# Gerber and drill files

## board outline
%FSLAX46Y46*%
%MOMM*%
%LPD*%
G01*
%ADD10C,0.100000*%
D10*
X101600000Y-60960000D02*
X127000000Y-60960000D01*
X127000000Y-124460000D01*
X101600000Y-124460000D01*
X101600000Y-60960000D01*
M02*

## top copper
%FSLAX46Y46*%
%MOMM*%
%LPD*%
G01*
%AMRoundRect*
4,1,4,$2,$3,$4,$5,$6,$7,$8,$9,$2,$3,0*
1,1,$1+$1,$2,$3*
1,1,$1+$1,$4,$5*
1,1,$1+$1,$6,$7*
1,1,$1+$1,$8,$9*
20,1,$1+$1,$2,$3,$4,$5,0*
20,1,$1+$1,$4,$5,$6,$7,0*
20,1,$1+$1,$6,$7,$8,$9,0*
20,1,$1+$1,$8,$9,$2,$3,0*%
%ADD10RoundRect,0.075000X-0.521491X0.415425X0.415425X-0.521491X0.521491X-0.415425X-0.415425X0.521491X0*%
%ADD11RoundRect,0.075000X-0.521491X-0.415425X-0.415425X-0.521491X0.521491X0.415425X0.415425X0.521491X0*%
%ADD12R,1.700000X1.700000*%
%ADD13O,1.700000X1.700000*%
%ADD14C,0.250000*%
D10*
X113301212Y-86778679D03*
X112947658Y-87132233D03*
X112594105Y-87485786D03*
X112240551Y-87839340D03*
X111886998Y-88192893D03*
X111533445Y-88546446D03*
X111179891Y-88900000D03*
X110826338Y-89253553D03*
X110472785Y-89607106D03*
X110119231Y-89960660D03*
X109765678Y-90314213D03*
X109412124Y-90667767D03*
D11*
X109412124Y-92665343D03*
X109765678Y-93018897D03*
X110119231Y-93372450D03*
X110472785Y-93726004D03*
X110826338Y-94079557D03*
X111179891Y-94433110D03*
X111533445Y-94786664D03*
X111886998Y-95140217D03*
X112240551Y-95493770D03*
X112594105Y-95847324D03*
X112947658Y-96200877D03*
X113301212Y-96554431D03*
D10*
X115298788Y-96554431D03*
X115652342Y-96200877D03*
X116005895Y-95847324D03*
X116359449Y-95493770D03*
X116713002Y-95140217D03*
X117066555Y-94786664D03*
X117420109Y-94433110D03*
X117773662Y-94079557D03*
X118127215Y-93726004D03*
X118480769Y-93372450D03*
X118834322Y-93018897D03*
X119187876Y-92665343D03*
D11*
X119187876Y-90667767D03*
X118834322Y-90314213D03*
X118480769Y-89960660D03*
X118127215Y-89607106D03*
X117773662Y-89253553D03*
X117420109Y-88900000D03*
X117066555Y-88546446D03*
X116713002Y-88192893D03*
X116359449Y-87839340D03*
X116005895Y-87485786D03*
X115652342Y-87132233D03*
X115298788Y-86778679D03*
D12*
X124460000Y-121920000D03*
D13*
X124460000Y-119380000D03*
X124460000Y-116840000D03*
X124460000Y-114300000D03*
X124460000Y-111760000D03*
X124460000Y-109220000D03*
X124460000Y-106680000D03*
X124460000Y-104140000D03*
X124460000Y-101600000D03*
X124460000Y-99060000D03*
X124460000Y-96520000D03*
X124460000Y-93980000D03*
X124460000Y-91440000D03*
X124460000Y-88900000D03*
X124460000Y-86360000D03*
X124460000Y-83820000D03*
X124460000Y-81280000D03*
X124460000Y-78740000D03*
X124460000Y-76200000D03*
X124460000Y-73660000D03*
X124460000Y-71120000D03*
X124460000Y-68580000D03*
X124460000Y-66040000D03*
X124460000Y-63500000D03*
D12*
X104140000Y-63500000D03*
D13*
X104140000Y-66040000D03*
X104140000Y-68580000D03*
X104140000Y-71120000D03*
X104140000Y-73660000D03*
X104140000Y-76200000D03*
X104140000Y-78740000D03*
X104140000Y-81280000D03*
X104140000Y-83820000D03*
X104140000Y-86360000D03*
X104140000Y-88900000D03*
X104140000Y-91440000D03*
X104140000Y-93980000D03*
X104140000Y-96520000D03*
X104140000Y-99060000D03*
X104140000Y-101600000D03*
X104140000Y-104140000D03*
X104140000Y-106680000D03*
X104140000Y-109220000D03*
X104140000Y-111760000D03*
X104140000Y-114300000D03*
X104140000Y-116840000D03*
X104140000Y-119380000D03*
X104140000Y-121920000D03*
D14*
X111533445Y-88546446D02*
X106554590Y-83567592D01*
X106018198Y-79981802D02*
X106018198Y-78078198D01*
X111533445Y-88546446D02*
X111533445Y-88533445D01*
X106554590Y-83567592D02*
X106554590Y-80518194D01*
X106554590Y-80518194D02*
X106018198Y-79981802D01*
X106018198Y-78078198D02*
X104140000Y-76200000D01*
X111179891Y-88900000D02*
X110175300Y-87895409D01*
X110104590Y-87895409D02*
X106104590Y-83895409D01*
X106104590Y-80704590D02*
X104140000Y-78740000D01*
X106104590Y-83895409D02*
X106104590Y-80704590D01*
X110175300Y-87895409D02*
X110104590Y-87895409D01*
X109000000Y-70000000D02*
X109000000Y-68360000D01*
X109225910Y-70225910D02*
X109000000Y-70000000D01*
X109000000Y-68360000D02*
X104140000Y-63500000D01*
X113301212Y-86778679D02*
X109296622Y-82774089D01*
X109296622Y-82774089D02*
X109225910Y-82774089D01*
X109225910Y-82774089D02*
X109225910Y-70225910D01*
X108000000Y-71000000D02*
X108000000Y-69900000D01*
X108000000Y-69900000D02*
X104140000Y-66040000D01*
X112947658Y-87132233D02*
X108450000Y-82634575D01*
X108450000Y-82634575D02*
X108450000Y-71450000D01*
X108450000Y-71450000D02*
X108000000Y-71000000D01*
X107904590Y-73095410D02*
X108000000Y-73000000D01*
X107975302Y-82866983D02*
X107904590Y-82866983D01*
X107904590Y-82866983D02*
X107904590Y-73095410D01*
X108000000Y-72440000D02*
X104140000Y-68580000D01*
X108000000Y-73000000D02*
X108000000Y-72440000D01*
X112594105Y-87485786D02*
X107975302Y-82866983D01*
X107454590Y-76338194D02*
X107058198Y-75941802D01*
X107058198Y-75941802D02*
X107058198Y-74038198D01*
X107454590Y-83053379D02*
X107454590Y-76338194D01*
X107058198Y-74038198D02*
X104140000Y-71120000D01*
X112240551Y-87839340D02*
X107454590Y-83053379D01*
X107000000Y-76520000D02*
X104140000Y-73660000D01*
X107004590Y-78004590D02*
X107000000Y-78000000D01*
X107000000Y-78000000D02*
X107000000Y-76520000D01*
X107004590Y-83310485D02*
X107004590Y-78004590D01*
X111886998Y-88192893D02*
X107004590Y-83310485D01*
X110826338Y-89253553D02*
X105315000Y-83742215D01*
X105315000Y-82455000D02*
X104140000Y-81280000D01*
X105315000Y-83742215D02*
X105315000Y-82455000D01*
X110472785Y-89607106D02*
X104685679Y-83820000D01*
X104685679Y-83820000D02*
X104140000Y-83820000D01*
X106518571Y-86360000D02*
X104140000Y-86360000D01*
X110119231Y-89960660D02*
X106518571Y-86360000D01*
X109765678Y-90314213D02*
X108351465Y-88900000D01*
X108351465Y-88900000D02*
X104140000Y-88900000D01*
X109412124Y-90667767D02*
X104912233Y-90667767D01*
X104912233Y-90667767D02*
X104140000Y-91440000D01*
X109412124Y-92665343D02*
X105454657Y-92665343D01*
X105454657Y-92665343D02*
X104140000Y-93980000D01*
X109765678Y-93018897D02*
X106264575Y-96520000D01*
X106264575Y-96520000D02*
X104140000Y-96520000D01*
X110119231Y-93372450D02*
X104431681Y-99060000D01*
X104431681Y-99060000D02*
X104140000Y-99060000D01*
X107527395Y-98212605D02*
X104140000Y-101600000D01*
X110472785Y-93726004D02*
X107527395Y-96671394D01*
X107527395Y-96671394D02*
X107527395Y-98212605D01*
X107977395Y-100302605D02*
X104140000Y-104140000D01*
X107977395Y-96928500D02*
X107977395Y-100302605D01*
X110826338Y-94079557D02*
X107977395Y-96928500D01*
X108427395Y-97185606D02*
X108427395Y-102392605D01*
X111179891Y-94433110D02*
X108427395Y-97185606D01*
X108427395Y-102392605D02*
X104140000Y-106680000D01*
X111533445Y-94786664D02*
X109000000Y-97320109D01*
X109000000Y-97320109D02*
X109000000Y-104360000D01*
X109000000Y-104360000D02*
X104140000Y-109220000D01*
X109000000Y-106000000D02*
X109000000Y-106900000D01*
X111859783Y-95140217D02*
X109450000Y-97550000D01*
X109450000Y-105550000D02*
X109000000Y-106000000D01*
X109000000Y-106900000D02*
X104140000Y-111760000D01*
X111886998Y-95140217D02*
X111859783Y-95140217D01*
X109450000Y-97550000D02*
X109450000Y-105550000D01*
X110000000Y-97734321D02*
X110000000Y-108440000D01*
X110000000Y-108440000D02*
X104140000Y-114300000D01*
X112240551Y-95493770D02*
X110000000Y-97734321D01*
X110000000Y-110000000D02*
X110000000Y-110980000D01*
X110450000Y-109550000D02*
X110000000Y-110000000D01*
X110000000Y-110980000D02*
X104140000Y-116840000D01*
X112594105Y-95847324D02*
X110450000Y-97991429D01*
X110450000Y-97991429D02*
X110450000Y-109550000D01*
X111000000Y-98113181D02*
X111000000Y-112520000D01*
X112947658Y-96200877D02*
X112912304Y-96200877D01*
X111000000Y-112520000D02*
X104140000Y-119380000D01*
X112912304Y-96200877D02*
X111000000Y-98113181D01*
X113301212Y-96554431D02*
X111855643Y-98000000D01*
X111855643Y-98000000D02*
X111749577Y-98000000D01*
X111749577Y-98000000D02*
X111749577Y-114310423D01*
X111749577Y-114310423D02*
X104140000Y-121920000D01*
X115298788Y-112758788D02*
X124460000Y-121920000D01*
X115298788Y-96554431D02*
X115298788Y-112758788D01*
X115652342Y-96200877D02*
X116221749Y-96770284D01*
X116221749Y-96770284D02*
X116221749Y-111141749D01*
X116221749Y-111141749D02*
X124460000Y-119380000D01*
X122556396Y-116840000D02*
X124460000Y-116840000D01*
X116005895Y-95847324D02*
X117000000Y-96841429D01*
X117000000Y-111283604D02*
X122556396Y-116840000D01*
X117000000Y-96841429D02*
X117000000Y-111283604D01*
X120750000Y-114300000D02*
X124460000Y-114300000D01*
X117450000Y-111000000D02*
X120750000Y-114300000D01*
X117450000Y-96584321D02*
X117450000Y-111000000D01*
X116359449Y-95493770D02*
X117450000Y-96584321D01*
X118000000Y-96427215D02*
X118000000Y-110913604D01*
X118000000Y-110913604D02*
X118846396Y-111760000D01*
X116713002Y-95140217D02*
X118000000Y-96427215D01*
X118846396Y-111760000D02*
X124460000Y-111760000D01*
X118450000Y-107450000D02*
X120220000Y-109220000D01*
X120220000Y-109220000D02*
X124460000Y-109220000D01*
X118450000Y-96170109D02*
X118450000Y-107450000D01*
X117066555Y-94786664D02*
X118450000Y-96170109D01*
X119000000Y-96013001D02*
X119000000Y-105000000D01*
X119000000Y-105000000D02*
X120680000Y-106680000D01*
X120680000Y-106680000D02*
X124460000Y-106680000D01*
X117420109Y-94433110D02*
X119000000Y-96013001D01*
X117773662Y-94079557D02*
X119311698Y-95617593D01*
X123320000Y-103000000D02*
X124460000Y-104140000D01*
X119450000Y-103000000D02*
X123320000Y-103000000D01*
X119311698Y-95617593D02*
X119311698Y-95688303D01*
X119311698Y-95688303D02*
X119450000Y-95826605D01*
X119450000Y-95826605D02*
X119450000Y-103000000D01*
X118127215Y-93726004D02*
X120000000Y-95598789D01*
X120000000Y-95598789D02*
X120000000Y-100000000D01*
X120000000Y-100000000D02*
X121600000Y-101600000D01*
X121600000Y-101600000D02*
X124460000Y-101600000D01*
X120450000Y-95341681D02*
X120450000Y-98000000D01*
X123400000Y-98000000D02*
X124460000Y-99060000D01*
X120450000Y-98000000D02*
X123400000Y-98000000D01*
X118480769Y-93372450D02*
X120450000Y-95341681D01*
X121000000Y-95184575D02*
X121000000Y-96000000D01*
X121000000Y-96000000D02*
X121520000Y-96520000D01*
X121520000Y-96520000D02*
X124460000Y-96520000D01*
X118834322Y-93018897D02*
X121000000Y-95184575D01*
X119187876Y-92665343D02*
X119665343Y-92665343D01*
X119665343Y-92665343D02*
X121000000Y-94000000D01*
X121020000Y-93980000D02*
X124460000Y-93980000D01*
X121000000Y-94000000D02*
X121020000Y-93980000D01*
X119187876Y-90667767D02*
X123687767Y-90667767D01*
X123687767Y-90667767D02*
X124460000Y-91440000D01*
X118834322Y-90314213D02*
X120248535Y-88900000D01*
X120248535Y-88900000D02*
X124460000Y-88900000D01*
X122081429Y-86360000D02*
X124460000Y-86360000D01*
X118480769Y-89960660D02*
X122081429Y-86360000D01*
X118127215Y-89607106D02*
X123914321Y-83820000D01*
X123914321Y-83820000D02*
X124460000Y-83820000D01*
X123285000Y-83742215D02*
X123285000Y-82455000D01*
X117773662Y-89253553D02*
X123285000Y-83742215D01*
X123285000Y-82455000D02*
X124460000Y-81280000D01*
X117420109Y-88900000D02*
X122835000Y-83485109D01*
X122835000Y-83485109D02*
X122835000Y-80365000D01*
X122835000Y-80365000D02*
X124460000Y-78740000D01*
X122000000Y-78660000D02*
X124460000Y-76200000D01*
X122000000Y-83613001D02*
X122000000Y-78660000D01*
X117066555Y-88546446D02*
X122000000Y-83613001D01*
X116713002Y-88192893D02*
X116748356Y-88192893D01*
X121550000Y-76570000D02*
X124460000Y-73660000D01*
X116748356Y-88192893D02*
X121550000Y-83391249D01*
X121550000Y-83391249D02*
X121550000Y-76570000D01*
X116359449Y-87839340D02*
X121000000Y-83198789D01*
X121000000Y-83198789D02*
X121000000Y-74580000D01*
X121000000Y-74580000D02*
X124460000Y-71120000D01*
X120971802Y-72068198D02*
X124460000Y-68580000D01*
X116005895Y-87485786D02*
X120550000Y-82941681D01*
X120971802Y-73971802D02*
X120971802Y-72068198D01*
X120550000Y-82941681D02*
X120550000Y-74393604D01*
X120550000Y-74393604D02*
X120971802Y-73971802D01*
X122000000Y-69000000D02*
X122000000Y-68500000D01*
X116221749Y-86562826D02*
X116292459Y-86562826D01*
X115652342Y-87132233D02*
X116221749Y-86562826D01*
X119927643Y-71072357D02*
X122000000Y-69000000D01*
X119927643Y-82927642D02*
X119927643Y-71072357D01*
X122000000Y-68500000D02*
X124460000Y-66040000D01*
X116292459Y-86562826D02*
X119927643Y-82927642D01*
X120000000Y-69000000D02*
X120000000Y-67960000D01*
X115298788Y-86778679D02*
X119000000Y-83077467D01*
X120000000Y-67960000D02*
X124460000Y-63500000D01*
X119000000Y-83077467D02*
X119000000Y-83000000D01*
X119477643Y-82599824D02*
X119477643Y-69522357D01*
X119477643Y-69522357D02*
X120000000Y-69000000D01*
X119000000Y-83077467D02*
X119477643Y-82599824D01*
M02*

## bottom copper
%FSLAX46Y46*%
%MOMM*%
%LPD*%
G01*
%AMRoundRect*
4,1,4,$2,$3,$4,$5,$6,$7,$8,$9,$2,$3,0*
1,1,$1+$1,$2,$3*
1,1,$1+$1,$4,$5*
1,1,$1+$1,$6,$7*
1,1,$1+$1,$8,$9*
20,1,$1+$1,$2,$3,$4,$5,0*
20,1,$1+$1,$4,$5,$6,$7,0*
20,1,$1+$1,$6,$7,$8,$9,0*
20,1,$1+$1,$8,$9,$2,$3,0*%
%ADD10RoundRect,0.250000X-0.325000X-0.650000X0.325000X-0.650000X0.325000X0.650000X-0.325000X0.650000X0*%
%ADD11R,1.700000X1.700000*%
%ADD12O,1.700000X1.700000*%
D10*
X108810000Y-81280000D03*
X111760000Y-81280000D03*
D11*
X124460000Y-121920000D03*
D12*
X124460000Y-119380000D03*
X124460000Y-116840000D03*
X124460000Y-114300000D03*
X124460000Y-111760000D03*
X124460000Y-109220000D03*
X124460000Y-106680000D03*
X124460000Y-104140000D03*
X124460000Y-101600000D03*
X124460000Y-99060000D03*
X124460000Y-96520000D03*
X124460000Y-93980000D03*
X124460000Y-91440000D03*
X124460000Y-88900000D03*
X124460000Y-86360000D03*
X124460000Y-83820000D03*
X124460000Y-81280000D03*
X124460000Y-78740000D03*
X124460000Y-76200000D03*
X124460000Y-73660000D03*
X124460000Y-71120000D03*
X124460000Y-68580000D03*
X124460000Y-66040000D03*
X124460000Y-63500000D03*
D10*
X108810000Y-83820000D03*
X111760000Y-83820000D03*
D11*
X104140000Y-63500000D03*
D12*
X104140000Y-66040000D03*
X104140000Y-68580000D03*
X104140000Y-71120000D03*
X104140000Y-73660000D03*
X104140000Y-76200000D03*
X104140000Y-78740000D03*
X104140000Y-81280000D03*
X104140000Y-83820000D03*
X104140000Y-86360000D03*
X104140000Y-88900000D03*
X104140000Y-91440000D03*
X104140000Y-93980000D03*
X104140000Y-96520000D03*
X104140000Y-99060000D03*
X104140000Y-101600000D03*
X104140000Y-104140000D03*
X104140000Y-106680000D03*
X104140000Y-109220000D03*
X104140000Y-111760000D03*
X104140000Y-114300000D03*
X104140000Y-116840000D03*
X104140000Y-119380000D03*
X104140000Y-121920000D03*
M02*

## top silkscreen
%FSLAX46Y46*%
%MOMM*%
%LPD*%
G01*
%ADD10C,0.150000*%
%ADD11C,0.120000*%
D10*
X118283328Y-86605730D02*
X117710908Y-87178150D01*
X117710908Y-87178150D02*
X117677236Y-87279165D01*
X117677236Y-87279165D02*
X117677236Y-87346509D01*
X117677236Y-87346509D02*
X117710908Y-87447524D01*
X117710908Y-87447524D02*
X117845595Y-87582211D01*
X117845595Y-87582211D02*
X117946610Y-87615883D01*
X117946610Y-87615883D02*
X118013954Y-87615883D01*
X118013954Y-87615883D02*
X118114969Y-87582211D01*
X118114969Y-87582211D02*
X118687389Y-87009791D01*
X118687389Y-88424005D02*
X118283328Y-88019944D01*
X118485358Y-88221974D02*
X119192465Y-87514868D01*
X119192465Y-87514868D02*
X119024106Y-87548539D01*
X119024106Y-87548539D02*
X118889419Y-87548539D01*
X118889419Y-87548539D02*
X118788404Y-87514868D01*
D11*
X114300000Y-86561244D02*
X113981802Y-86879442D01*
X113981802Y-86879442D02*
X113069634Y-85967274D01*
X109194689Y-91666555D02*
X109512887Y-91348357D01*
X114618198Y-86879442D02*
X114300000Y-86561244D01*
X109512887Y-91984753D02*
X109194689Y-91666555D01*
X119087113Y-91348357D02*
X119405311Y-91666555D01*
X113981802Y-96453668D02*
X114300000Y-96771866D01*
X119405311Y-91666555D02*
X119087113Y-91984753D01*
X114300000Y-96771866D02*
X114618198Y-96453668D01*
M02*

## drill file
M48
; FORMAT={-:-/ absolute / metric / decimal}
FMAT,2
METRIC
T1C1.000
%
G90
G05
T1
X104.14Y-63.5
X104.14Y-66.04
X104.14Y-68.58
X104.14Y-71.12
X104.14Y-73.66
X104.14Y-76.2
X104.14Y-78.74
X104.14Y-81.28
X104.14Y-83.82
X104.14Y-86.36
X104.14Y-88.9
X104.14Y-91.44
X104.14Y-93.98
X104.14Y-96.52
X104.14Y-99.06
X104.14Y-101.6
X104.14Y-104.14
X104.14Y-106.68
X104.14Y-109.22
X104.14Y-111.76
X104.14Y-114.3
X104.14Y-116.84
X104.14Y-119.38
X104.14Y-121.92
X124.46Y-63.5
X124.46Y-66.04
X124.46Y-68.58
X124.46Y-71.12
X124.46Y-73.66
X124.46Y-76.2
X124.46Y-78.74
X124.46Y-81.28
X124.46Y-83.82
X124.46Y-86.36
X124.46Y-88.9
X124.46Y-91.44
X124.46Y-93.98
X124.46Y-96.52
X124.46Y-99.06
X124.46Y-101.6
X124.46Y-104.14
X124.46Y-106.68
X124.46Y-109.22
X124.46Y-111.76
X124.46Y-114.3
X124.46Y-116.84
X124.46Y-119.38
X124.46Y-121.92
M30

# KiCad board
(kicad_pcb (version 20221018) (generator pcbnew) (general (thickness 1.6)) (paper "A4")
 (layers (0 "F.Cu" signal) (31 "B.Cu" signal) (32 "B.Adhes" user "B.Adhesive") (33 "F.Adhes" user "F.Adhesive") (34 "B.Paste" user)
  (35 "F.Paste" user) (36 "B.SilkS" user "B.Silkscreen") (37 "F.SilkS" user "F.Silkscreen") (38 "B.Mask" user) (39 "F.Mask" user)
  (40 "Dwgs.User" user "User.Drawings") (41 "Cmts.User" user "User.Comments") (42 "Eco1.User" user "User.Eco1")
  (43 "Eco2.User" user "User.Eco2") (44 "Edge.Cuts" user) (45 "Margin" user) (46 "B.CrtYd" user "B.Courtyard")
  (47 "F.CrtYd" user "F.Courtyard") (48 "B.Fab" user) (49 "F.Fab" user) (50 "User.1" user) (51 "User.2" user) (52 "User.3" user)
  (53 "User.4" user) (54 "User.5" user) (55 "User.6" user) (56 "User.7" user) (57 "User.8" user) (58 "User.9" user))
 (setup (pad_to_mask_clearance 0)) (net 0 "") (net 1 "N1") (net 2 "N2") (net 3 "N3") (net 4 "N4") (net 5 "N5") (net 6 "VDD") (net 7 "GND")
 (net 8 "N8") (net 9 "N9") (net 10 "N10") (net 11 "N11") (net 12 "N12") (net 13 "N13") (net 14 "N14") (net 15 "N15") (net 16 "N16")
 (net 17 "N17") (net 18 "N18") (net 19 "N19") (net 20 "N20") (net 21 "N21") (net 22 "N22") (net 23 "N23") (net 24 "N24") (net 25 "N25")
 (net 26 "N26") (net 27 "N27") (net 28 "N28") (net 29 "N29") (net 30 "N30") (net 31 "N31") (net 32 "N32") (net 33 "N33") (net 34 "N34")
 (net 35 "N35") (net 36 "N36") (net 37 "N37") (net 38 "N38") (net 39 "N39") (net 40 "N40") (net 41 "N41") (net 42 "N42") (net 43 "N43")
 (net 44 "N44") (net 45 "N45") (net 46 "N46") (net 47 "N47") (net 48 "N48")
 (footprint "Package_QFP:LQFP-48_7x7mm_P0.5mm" (layer "F.Cu") (at 114.3 91.666555 -45)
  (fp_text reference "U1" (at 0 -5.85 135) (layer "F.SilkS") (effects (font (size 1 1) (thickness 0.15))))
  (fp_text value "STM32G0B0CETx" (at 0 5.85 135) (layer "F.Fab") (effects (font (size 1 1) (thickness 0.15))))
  (fp_line (start -3.61 -3.61) (end -3.61 -3.16) (stroke (width 0.12) (type solid)) (layer "F.SilkS"))
  (fp_line (start -3.61 -3.16) (end -4.9 -3.16) (stroke (width 0.12) (type solid)) (layer "F.SilkS"))
  (fp_line (start -3.61 3.61) (end -3.61 3.16) (stroke (width 0.12) (type solid)) (layer "F.SilkS"))
  (fp_line (start -3.16 -3.61) (end -3.61 -3.61) (stroke (width 0.12) (type solid)) (layer "F.SilkS"))
  (fp_line (start -3.16 3.61) (end -3.61 3.61) (stroke (width 0.12) (type solid)) (layer "F.SilkS"))
  (fp_line (start 3.16 -3.61) (end 3.61 -3.61) (stroke (width 0.12) (type solid)) (layer "F.SilkS"))
  (fp_line (start 3.16 3.61) (end 3.61 3.61) (stroke (width 0.12) (type solid)) (layer "F.SilkS"))
  (fp_line (start 3.61 -3.61) (end 3.61 -3.16) (stroke (width 0.12) (type solid)) (layer "F.SilkS"))
  (fp_line (start 3.61 3.61) (end 3.61 3.16) (stroke (width 0.12) (type solid)) (layer "F.SilkS"))
  (pad "1" smd roundrect (at -4.1625 -2.75 315) (size 1.475 0.3) (layers "F.Cu" "F.Paste" "F.Mask") (roundrect_rratio 0.25) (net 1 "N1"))
  (pad "2" smd roundrect (at -4.1625 -2.25 315) (size 1.475 0.3) (layers "F.Cu" "F.Paste" "F.Mask") (roundrect_rratio 0.25) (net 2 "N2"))
  (pad "3" smd roundrect (at -4.1625 -1.75 315) (size 1.475 0.3) (layers "F.Cu" "F.Paste" "F.Mask") (roundrect_rratio 0.25) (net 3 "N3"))
  (pad "4" smd roundrect (at -4.1625 -1.25 315) (size 1.475 0.3) (layers "F.Cu" "F.Paste" "F.Mask") (roundrect_rratio 0.25) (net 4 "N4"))
  (pad "5" smd roundrect (at -4.1625 -0.75 315) (size 1.475 0.3) (layers "F.Cu" "F.Paste" "F.Mask") (roundrect_rratio 0.25) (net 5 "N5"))
  (pad "6" smd roundrect (at -4.1625 -0.25 315) (size 1.475 0.3) (layers "F.Cu" "F.Paste" "F.Mask") (roundrect_rratio 0.25) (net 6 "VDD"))
  (pad "7" smd roundrect (at -4.1625 0.25 315) (size 1.475 0.3) (layers "F.Cu" "F.Paste" "F.Mask") (roundrect_rratio 0.25) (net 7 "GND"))
  (pad "8" smd roundrect (at -4.1625 0.75 315) (size 1.475 0.3) (layers "F.Cu" "F.Paste" "F.Mask") (roundrect_rratio 0.25) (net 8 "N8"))
  (pad "9" smd roundrect (at -4.1625 1.25 315) (size 1.475 0.3) (layers "F.Cu" "F.Paste" "F.Mask") (roundrect_rratio 0.25) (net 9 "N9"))
  (pad "10" smd roundrect (at -4.1625 1.75 315) (size 1.475 0.3) (layers "F.Cu" "F.Paste" "F.Mask") (roundrect_rratio 0.25) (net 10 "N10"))
  (pad "11" smd roundrect (at -4.1625 2.25 315) (size 1.475 0.3) (layers "F.Cu" "F.Paste" "F.Mask") (roundrect_rratio 0.25) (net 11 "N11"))
  (pad "12" smd roundrect (at -4.1625 2.75 315) (size 1.475 0.3) (layers "F.Cu" "F.Paste" "F.Mask") (roundrect_rratio 0.25) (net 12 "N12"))
  (pad "13" smd roundrect (at -2.75 4.1625 315) (size 0.3 1.475) (layers "F.Cu" "F.Paste" "F.Mask") (roundrect_rratio 0.25) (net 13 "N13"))
  (pad "14" smd roundrect (at -2.25 4.1625 315) (size 0.3 1.475) (layers "F.Cu" "F.Paste" "F.Mask") (roundrect_rratio 0.25) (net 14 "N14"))
  (pad "15" smd roundrect (at -1.75 4.1625 315) (size 0.3 1.475) (layers "F.Cu" "F.Paste" "F.Mask") (roundrect_rratio 0.25) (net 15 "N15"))
  (pad "16" smd roundrect (at -1.25 4.1625 315) (size 0.3 1.475) (layers "F.Cu" "F.Paste" "F.Mask") (roundrect_rratio 0.25) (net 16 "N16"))
  (pad "17" smd roundrect (at -0.75 4.1625 315) (size 0.3 1.475) (layers "F.Cu" "F.Paste" "F.Mask") (roundrect_rratio 0.25) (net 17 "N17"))
  (pad "18" smd roundrect (at -0.25 4.1625 315) (size 0.3 1.475) (layers "F.Cu" "F.Paste" "F.Mask") (roundrect_rratio 0.25) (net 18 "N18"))
  (pad "19" smd roundrect (at 0.25 4.1625 315) (size 0.3 1.475) (layers "F.Cu" "F.Paste" "F.Mask") (roundrect_rratio 0.25) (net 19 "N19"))
  (pad "20" smd roundrect (at 0.75 4.1625 315) (size 0.3 1.475) (layers "F.Cu" "F.Paste" "F.Mask") (roundrect_rratio 0.25) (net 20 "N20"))
  (pad "21" smd roundrect (at 1.25 4.1625 315) (size 0.3 1.475) (layers "F.Cu" "F.Paste" "F.Mask") (roundrect_rratio 0.25) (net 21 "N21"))
  (pad "22" smd roundrect (at 1.75 4.1625 315) (size 0.3 1.475) (layers "F.Cu" "F.Paste" "F.Mask") (roundrect_rratio 0.25) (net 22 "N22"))
  (pad "23" smd roundrect (at 2.25 4.1625 315) (size 0.3 1.475) (layers "F.Cu" "F.Paste" "F.Mask") (roundrect_rratio 0.25) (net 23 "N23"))
  (pad "24" smd roundrect (at 2.75 4.1625 315) (size 0.3 1.475) (layers "F.Cu" "F.Paste" "F.Mask") (roundrect_rratio 0.25) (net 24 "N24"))
  (pad "25" smd roundrect (at 4.1625 2.75 315) (size 1.475 0.3) (layers "F.Cu" "F.Paste" "F.Mask") (roundrect_rratio 0.25) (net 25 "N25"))
  (pad "26" smd roundrect (at 4.1625 2.25 315) (size 1.475 0.3) (layers "F.Cu" "F.Paste" "F.Mask") (roundrect_rratio 0.25) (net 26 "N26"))
  (pad "27" smd roundrect (at 4.1625 1.75 315) (size 1.475 0.3) (layers "F.Cu" "F.Paste" "F.Mask") (roundrect_rratio 0.25) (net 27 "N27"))
  (pad "28" smd roundrect (at 4.1625 1.25 315) (size 1.475 0.3) (layers "F.Cu" "F.Paste" "F.Mask") (roundrect_rratio 0.25) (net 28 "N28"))
  (pad "29" smd roundrect (at 4.1625 0.75 315) (size 1.475 0.3) (layers "F.Cu" "F.Paste" "F.Mask") (roundrect_rratio 0.25) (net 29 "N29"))
  (pad "30" smd roundrect (at 4.1625 0.25 315) (size 1.475 0.3) (layers "F.Cu" "F.Paste" "F.Mask") (roundrect_rratio 0.25) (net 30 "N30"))
  (pad "31" smd roundrect (at 4.1625 -0.25 315) (size 1.475 0.3) (layers "F.Cu" "F.Paste" "F.Mask") (roundrect_rratio 0.25) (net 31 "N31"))
  (pad "32" smd roundrect (at 4.1625 -0.75 315) (size 1.475 0.3) (layers "F.Cu" "F.Paste" "F.Mask") (roundrect_rratio 0.25) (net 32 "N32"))
  (pad "33" smd roundrect (at 4.1625 -1.25 315) (size 1.475 0.3) (layers "F.Cu" "F.Paste" "F.Mask") (roundrect_rratio 0.25) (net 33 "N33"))
  (pad "34" smd roundrect (at 4.1625 -1.75 315) (size 1.475 0.3) (layers "F.Cu" "F.Paste" "F.Mask") (roundrect_rratio 0.25) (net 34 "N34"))
  (pad "35" smd roundrect (at 4.1625 -2.25 315) (size 1.475 0.3) (layers "F.Cu" "F.Paste" "F.Mask") (roundrect_rratio 0.25) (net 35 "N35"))
  (pad "36" smd roundrect (at 4.1625 -2.75 315) (size 1.475 0.3) (layers "F.Cu" "F.Paste" "F.Mask") (roundrect_rratio 0.25) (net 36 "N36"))
  (pad "37" smd roundrect (at 2.75 -4.1625 315) (size 0.3 1.475) (layers "F.Cu" "F.Paste" "F.Mask") (roundrect_rratio 0.25) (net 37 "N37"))
  (pad "38" smd roundrect (at 2.25 -4.1625 315) (size 0.3 1.475) (layers "F.Cu" "F.Paste" "F.Mask") (roundrect_rratio 0.25) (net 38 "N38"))
  (pad "39" smd roundrect (at 1.75 -4.1625 315) (size 0.3 1.475) (layers "F.Cu" "F.Paste" "F.Mask") (roundrect_rratio 0.25) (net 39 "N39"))
  (pad "40" smd roundrect (at 1.25 -4.1625 315) (size 0.3 1.475) (layers "F.Cu" "F.Paste" "F.Mask") (roundrect_rratio 0.25) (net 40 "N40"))
  (pad "41" smd roundrect (at 0.75 -4.1625 315) (size 0.3 1.475) (layers "F.Cu" "F.Paste" "F.Mask") (roundrect_rratio 0.25) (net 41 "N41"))
  (pad "42" smd roundrect (at 0.25 -4.1625 315) (size 0.3 1.475) (layers "F.Cu" "F.Paste" "F.Mask") (roundrect_rratio 0.25) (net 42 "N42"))
  (pad "43" smd roundrect (at -0.25 -4.1625 315) (size 0.3 1.475) (layers "F.Cu" "F.Paste" "F.Mask") (roundrect_rratio 0.25) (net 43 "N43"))
  (pad "44" smd roundrect (at -0.75 -4.1625 315) (size 0.3 1.475) (layers "F.Cu" "F.Paste" "F.Mask") (roundrect_rratio 0.25) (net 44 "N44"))
  (pad "45" smd roundrect (at -1.25 -4.1625 315) (size 0.3 1.475) (layers "F.Cu" "F.Paste" "F.Mask") (roundrect_rratio 0.25) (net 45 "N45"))
  (pad "46" smd roundrect (at -1.75 -4.1625 315) (size 0.3 1.475) (layers "F.Cu" "F.Paste" "F.Mask") (roundrect_rratio 0.25) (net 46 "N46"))
  (pad "47" smd roundrect (at -2.25 -4.1625 315) (size 0.3 1.475) (layers "F.Cu" "F.Paste" "F.Mask") (roundrect_rratio 0.25) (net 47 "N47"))
  (pad "48" smd roundrect (at -2.75 -4.1625 315) (size 0.3 1.475) (layers "F.Cu" "F.Paste" "F.Mask") (roundrect_rratio 0.25) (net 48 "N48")))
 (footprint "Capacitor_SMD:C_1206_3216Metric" (layer "B.Cu") (at 110.285 81.28)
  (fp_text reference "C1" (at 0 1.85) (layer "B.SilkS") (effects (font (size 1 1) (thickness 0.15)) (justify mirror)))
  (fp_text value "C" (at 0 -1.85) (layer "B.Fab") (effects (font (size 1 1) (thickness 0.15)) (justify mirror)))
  (pad "1" smd roundrect (at -1.475 0) (size 1.15 1.8) (layers "B.Cu" "B.Paste" "B.Mask") (roundrect_rratio 0.2173913043) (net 6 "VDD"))
  (pad "2" smd roundrect (at 1.475 0) (size 1.15 1.8) (layers "B.Cu" "B.Paste" "B.Mask") (roundrect_rratio 0.2173913043) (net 7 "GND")))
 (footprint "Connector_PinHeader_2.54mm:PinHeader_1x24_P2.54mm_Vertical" (layer "B.Cu") (at 124.46 121.92)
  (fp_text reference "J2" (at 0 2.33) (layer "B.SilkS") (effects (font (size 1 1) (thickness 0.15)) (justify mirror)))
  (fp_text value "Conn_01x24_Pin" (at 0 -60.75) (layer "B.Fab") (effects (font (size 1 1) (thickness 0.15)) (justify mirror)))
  (pad "1" thru_hole rect (at 0 0) (size 1.7 1.7) (drill 1) (layers "*.Cu" "*.Mask") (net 25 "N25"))
  (pad "2" thru_hole oval (at 0 -2.54) (size 1.7 1.7) (drill 1) (layers "*.Cu" "*.Mask") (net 26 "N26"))
  (pad "3" thru_hole oval (at 0 -5.08) (size 1.7 1.7) (drill 1) (layers "*.Cu" "*.Mask") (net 27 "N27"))
  (pad "4" thru_hole oval (at 0 -7.62) (size 1.7 1.7) (drill 1) (layers "*.Cu" "*.Mask") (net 28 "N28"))
  (pad "5" thru_hole oval (at 0 -10.16) (size 1.7 1.7) (drill 1) (layers "*.Cu" "*.Mask") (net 29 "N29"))
  (pad "6" thru_hole oval (at 0 -12.7) (size 1.7 1.7) (drill 1) (layers "*.Cu" "*.Mask") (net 30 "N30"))
  (pad "7" thru_hole oval (at 0 -15.24) (size 1.7 1.7) (drill 1) (layers "*.Cu" "*.Mask") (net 31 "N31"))
  (pad "8" thru_hole oval (at 0 -17.78) (size 1.7 1.7) (drill 1) (layers "*.Cu" "*.Mask") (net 32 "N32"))
  (pad "9" thru_hole oval (at 0 -20.32) (size 1.7 1.7) (drill 1) (layers "*.Cu" "*.Mask") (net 33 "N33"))
  (pad "10" thru_hole oval (at 0 -22.86) (size 1.7 1.7) (drill 1) (layers "*.Cu" "*.Mask") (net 34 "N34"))
  (pad "11" thru_hole oval (at 0 -25.4) (size 1.7 1.7) (drill 1) (layers "*.Cu" "*.Mask") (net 35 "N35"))
  (pad "12" thru_hole oval (at 0 -27.94) (size 1.7 1.7) (drill 1) (layers "*.Cu" "*.Mask") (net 36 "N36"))
  (pad "13" thru_hole oval (at 0 -30.48) (size 1.7 1.7) (drill 1) (layers "*.Cu" "*.Mask") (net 37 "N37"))
  (pad "14" thru_hole oval (at 0 -33.02) (size 1.7 1.7) (drill 1) (layers "*.Cu" "*.Mask") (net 38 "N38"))
  (pad "15" thru_hole oval (at 0 -35.56) (size 1.7 1.7) (drill 1) (layers "*.Cu" "*.Mask") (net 39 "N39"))
  (pad "16" thru_hole oval (at 0 -38.1) (size 1.7 1.7) (drill 1) (layers "*.Cu" "*.Mask") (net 40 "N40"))
  (pad "17" thru_hole oval (at 0 -40.64) (size 1.7 1.7) (drill 1) (layers "*.Cu" "*.Mask") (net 41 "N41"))
  (pad "18" thru_hole oval (at 0 -43.18) (size 1.7 1.7) (drill 1) (layers "*.Cu" "*.Mask") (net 42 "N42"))
  (pad "19" thru_hole oval (at 0 -45.72) (size 1.7 1.7) (drill 1) (layers "*.Cu" "*.Mask") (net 43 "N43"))
  (pad "20" thru_hole oval (at 0 -48.26) (size 1.7 1.7) (drill 1) (layers "*.Cu" "*.Mask") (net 44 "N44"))
  (pad "21" thru_hole oval (at 0 -50.8) (size 1.7 1.7) (drill 1) (layers "*.Cu" "*.Mask") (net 45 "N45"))
  (pad "22" thru_hole oval (at 0 -53.34) (size 1.7 1.7) (drill 1) (layers "*.Cu" "*.Mask") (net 46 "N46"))
  (pad "23" thru_hole oval (at 0 -55.88) (size 1.7 1.7) (drill 1) (layers "*.Cu" "*.Mask") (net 47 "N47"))
  (pad "24" thru_hole oval (at 0 -58.42) (size 1.7 1.7) (drill 1) (layers "*.Cu" "*.Mask") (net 48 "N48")))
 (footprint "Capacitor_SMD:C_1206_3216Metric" (layer "B.Cu") (at 110.285 83.82)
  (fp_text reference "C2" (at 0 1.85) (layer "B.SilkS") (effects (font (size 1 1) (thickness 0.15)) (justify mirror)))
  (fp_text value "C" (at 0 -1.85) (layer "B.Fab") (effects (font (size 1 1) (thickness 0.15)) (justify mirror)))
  (pad "1" smd roundrect (at -1.475 0) (size 1.15 1.8) (layers "B.Cu" "B.Paste" "B.Mask") (roundrect_rratio 0.2173913043) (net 6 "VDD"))
  (pad "2" smd roundrect (at 1.475 0) (size 1.15 1.8) (layers "B.Cu" "B.Paste" "B.Mask") (roundrect_rratio 0.2173913043) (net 7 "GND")))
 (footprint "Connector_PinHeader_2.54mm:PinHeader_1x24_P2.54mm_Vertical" (layer "B.Cu") (at 104.14 63.5 180)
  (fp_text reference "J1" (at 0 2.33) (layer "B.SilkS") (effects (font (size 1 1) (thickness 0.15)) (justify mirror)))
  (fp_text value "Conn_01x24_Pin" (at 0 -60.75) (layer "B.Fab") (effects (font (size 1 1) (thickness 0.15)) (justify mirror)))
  (pad "1" thru_hole rect (at 0 0 180) (size 1.7 1.7) (drill 1) (layers "*.Cu" "*.Mask") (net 1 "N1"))
  (pad "2" thru_hole oval (at 0 -2.54 180) (size 1.7 1.7) (drill 1) (layers "*.Cu" "*.Mask") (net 2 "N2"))
  (pad "3" thru_hole oval (at 0 -5.08 180) (size 1.7 1.7) (drill 1) (layers "*.Cu" "*.Mask") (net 3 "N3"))
  (pad "4" thru_hole oval (at 0 -7.62 180) (size 1.7 1.7) (drill 1) (layers "*.Cu" "*.Mask") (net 4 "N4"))
  (pad "5" thru_hole oval (at 0 -10.16 180) (size 1.7 1.7) (drill 1) (layers "*.Cu" "*.Mask") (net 5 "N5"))
  (pad "6" thru_hole oval (at 0 -12.7 180) (size 1.7 1.7) (drill 1) (layers "*.Cu" "*.Mask") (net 6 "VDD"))
  (pad "7" thru_hole oval (at 0 -15.24 180) (size 1.7 1.7) (drill 1) (layers "*.Cu" "*.Mask") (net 7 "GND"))
  (pad "8" thru_hole oval (at 0 -17.78 180) (size 1.7 1.7) (drill 1) (layers "*.Cu" "*.Mask") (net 8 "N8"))
  (pad "9" thru_hole oval (at 0 -20.32 180) (size 1.7 1.7) (drill 1) (layers "*.Cu" "*.Mask") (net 9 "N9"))
  (pad "10" thru_hole oval (at 0 -22.86 180) (size 1.7 1.7) (drill 1) (layers "*.Cu" "*.Mask") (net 10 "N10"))
  (pad "11" thru_hole oval (at 0 -25.4 180) (size 1.7 1.7) (drill 1) (layers "*.Cu" "*.Mask") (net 11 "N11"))
  (pad "12" thru_hole oval (at 0 -27.94 180) (size 1.7 1.7) (drill 1) (layers "*.Cu" "*.Mask") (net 12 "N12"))
  (pad "13" thru_hole oval (at 0 -30.48 180) (size 1.7 1.7) (drill 1) (layers "*.Cu" "*.Mask") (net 13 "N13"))
  (pad "14" thru_hole oval (at 0 -33.02 180) (size 1.7 1.7) (drill 1) (layers "*.Cu" "*.Mask") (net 14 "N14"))
  (pad "15" thru_hole oval (at 0 -35.56 180) (size 1.7 1.7) (drill 1) (layers "*.Cu" "*.Mask") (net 15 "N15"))
  (pad "16" thru_hole oval (at 0 -38.1 180) (size 1.7 1.7) (drill 1) (layers "*.Cu" "*.Mask") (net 16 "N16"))
  (pad "17" thru_hole oval (at 0 -40.64 180) (size 1.7 1.7) (drill 1) (layers "*.Cu" "*.Mask") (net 17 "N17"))
  (pad "18" thru_hole oval (at 0 -43.18 180) (size 1.7 1.7) (drill 1) (layers "*.Cu" "*.Mask") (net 18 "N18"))
  (pad "19" thru_hole oval (at 0 -45.72 180) (size 1.7 1.7) (drill 1) (layers "*.Cu" "*.Mask") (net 19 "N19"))
  (pad "20" thru_hole oval (at 0 -48.26 180) (size 1.7 1.7) (drill 1) (layers "*.Cu" "*.Mask") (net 20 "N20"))
  (pad "21" thru_hole oval (at 0 -50.8 180) (size 1.7 1.7) (drill 1) (layers "*.Cu" "*.Mask") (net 21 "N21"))
  (pad "22" thru_hole oval (at 0 -53.34 180) (size 1.7 1.7) (drill 1) (layers "*.Cu" "*.Mask") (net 22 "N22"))
  (pad "23" thru_hole oval (at 0 -55.88 180) (size 1.7 1.7) (drill 1) (layers "*.Cu" "*.Mask") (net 23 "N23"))
  (pad "24" thru_hole oval (at 0 -58.42 180) (size 1.7 1.7) (drill 1) (layers "*.Cu" "*.Mask") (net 24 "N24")))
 (gr_rect (start 101.6 60.96) (end 127 124.46) (stroke (width 0.1) (type default)) (fill none) (layer "Edge.Cuts"))
 (segment (start 111.533445 88.546446) (end 106.55459 83.567592) (width 0.25) (layer "F.Cu") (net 6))
 (segment (start 106.018198 79.981802) (end 106.018198 78.078198) (width 0.25) (layer "F.Cu") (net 6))
 (segment (start 111.533445 88.546446) (end 111.533445 88.533445) (width 0.25) (layer "F.Cu") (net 6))
 (segment (start 106.55459 83.567592) (end 106.55459 80.518194) (width 0.25) (layer "F.Cu") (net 6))
 (segment (start 106.55459 80.518194) (end 106.018198 79.981802) (width 0.25) (layer "F.Cu") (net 6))
 (segment (start 106.018198 78.078198) (end 104.14 76.2) (width 0.25) (layer "F.Cu") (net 6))
 (segment (start 111.179891 88.9) (end 110.1753 87.895409) (width 0.25) (layer "F.Cu") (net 7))
 (segment (start 110.10459 87.895409) (end 106.10459 83.895409) (width 0.25) (layer "F.Cu") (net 7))
 (segment (start 106.10459 80.70459) (end 104.14 78.74) (width 0.25) (layer "F.Cu") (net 7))
 (segment (start 106.10459 83.895409) (end 106.10459 80.70459) (width 0.25) (layer "F.Cu") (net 7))
 (segment (start 110.1753 87.895409) (end 110.10459 87.895409) (width 0.25) (layer "F.Cu") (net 7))
 (segment (start 109 70) (end 109 68.36) (width 0.25) (layer "F.Cu") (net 1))
 (segment (start 109.22591 70.22591) (end 109 70) (width 0.25) (layer "F.Cu") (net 1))
 (segment (start 109 68.36) (end 104.14 63.5) (width 0.25) (layer "F.Cu") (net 1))
 (segment (start 113.301212 86.778679) (end 109.296622 82.774089) (width 0.25) (layer "F.Cu") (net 1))
 (segment (start 109.296622 82.774089) (end 109.22591 82.774089) (width 0.25) (layer "F.Cu") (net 1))
 (segment (start 109.22591 82.774089) (end 109.22591 70.22591) (width 0.25) (layer "F.Cu") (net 1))
 (segment (start 108 71) (end 108 69.9) (width 0.25) (layer "F.Cu") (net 2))
 (segment (start 108 69.9) (end 104.14 66.04) (width 0.25) (layer "F.Cu") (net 2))
 (segment (start 112.947658 87.132233) (end 108.45 82.634575) (width 0.25) (layer "F.Cu") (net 2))
 (segment (start 108.45 82.634575) (end 108.45 71.45) (width 0.25) (layer "F.Cu") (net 2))
 (segment (start 108.45 71.45) (end 108 71) (width 0.25) (layer "F.Cu") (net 2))
 (segment (start 107.90459 73.09541) (end 108 73) (width 0.25) (layer "F.Cu") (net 3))
 (segment (start 107.975302 82.866983) (end 107.90459 82.866983) (width 0.25) (layer "F.Cu") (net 3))
 (segment (start 107.90459 82.866983) (end 107.90459 73.09541) (width 0.25) (layer "F.Cu") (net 3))
 (segment (start 108 72.44) (end 104.14 68.58) (width 0.25) (layer "F.Cu") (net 3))
 (segment (start 108 73) (end 108 72.44) (width 0.25) (layer "F.Cu") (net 3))
 (segment (start 112.594105 87.485786) (end 107.975302 82.866983) (width 0.25) (layer "F.Cu") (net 3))
 (segment (start 107.45459 76.338194) (end 107.058198 75.941802) (width 0.25) (layer "F.Cu") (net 4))
 (segment (start 107.058198 75.941802) (end 107.058198 74.038198) (width 0.25) (layer "F.Cu") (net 4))
 (segment (start 107.45459 83.053379) (end 107.45459 76.338194) (width 0.25) (layer "F.Cu") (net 4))
 (segment (start 107.058198 74.038198) (end 104.14 71.12) (width 0.25) (layer "F.Cu") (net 4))
 (segment (start 112.240551 87.83934) (end 107.45459 83.053379) (width 0.25) (layer "F.Cu") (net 4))
 (segment (start 107 76.52) (end 104.14 73.66) (width 0.25) (layer "F.Cu") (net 5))
 (segment (start 107.00459 78.00459) (end 107 78) (width 0.25) (layer "F.Cu") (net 5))
 (segment (start 107 78) (end 107 76.52) (width 0.25) (layer "F.Cu") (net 5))
 (segment (start 107.00459 83.310485) (end 107.00459 78.00459) (width 0.25) (layer "F.Cu") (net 5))
 (segment (start 111.886998 88.192893) (end 107.00459 83.310485) (width 0.25) (layer "F.Cu") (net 5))
 (segment (start 110.826338 89.253553) (end 105.315 83.742215) (width 0.25) (layer "F.Cu") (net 8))
 (segment (start 105.315 82.455) (end 104.14 81.28) (width 0.25) (layer "F.Cu") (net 8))
 (segment (start 105.315 83.742215) (end 105.315 82.455) (width 0.25) (layer "F.Cu") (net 8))
 (segment (start 110.472785 89.607106) (end 104.685679 83.82) (width 0.25) (layer "F.Cu") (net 9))
 (segment (start 104.685679 83.82) (end 104.14 83.82) (width 0.25) (layer "F.Cu") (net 9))
 (segment (start 106.518571 86.36) (end 104.14 86.36) (width 0.25) (layer "F.Cu") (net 10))
 (segment (start 110.119231 89.96066) (end 106.518571 86.36) (width 0.25) (layer "F.Cu") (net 10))
 (segment (start 109.765678 90.314213) (end 108.351465 88.9) (width 0.25) (layer "F.Cu") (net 11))
 (segment (start 108.351465 88.9) (end 104.14 88.9) (width 0.25) (layer "F.Cu") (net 11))
 (segment (start 109.412124 90.667767) (end 104.912233 90.667767) (width 0.25) (layer "F.Cu") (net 12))
 (segment (start 104.912233 90.667767) (end 104.14 91.44) (width 0.25) (layer "F.Cu") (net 12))
 (segment (start 109.412124 92.665343) (end 105.454657 92.665343) (width 0.25) (layer "F.Cu") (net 13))
 (segment (start 105.454657 92.665343) (end 104.14 93.98) (width 0.25) (layer "F.Cu") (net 13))
 (segment (start 109.765678 93.018897) (end 106.264575 96.52) (width 0.25) (layer "F.Cu") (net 14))
 (segment (start 106.264575 96.52) (end 104.14 96.52) (width 0.25) (layer "F.Cu") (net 14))
 (segment (start 110.119231 93.37245) (end 104.431681 99.06) (width 0.25) (layer "F.Cu") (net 15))
 (segment (start 104.431681 99.06) (end 104.14 99.06) (width 0.25) (layer "F.Cu") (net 15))
 (segment (start 107.527395 98.212605) (end 104.14 101.6) (width 0.25) (layer "F.Cu") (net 16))
 (segment (start 110.472785 93.726004) (end 107.527395 96.671394) (width 0.25) (layer "F.Cu") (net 16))
 (segment (start 107.527395 96.671394) (end 107.527395 98.212605) (width 0.25) (layer "F.Cu") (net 16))
 (segment (start 107.977395 100.302605) (end 104.14 104.14) (width 0.25) (layer "F.Cu") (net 17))
 (segment (start 107.977395 96.9285) (end 107.977395 100.302605) (width 0.25) (layer "F.Cu") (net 17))
 (segment (start 110.826338 94.079557) (end 107.977395 96.9285) (width 0.25) (layer "F.Cu") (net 17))
 (segment (start 108.427395 97.185606) (end 108.427395 102.392605) (width 0.25) (layer "F.Cu") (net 18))
 (segment (start 111.179891 94.43311) (end 108.427395 97.185606) (width 0.25) (layer "F.Cu") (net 18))
 (segment (start 108.427395 102.392605) (end 104.14 106.68) (width 0.25) (layer "F.Cu") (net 18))
 (segment (start 111.533445 94.786664) (end 109 97.320109) (width 0.25) (layer "F.Cu") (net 19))
 (segment (start 109 97.320109) (end 109 104.36) (width 0.25) (layer "F.Cu") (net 19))
 (segment (start 109 104.36) (end 104.14 109.22) (width 0.25) (layer "F.Cu") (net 19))
 (segment (start 109 106) (end 109 106.9) (width 0.25) (layer "F.Cu") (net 20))
 (segment (start 111.859783 95.140217) (end 109.45 97.55) (width 0.25) (layer "F.Cu") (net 20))
 (segment (start 109.45 105.55) (end 109 106) (width 0.25) (layer "F.Cu") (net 20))
 (segment (start 109 106.9) (end 104.14 111.76) (width 0.25) (layer "F.Cu") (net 20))
 (segment (start 111.886998 95.140217) (end 111.859783 95.140217) (width 0.25) (layer "F.Cu") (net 20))
 (segment (start 109.45 97.55) (end 109.45 105.55) (width 0.25) (layer "F.Cu") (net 20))
 (segment (start 110 97.734321) (end 110 108.44) (width 0.25) (layer "F.Cu") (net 21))
 (segment (start 110 108.44) (end 104.14 114.3) (width 0.25) (layer "F.Cu") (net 21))
 (segment (start 112.240551 95.49377) (end 110 97.734321) (width 0.25) (layer "F.Cu") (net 21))
 (segment (start 110 110) (end 110 110.98) (width 0.25) (layer "F.Cu") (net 22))
 (segment (start 110.45 109.55) (end 110 110) (width 0.25) (layer "F.Cu") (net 22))
 (segment (start 110 110.98) (end 104.14 116.84) (width 0.25) (layer "F.Cu") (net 22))
 (segment (start 112.594105 95.847324) (end 110.45 97.991429) (width 0.25) (layer "F.Cu") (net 22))
 (segment (start 110.45 97.991429) (end 110.45 109.55) (width 0.25) (layer "F.Cu") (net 22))
 (segment (start 111 98.113181) (end 111 112.52) (width 0.25) (layer "F.Cu") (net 23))
 (segment (start 112.947658 96.200877) (end 112.912304 96.200877) (width 0.25) (layer "F.Cu") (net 23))
 (segment (start 111 112.52) (end 104.14 119.38) (width 0.25) (layer "F.Cu") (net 23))
 (segment (start 112.912304 96.200877) (end 111 98.113181) (width 0.25) (layer "F.Cu") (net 23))
 (segment (start 113.301212 96.554431) (end 111.855643 98) (width 0.25) (layer "F.Cu") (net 24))
 (segment (start 111.855643 98) (end 111.749577 98) (width 0.25) (layer "F.Cu") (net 24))
 (segment (start 111.749577 98) (end 111.749577 114.310423) (width 0.25) (layer "F.Cu") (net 24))
 (segment (start 111.749577 114.310423) (end 104.14 121.92) (width 0.25) (layer "F.Cu") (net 24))
 (segment (start 115.298788 112.758788) (end 124.46 121.92) (width 0.25) (layer "F.Cu") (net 25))
 (segment (start 115.298788 96.554431) (end 115.298788 112.758788) (width 0.25) (layer "F.Cu") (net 25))
 (segment (start 115.652342 96.200877) (end 116.221749 96.770284) (width 0.25) (layer "F.Cu") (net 26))
 (segment (start 116.221749 96.770284) (end 116.221749 111.141749) (width 0.25) (layer "F.Cu") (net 26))
 (segment (start 116.221749 111.141749) (end 124.46 119.38) (width 0.25) (layer "F.Cu") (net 26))
 (segment (start 122.556396 116.84) (end 124.46 116.84) (width 0.25) (layer "F.Cu") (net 27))
 (segment (start 116.005895 95.847324) (end 117 96.841429) (width 0.25) (layer "F.Cu") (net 27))
 (segment (start 117 111.283604) (end 122.556396 116.84) (width 0.25) (layer "F.Cu") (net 27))
 (segment (start 117 96.841429) (end 117 111.283604) (width 0.25) (layer "F.Cu") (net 27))
 (segment (start 120.75 114.3) (end 124.46 114.3) (width 0.25) (layer "F.Cu") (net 28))
 (segment (start 117.45 111) (end 120.75 114.3) (width 0.25) (layer "F.Cu") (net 28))
 (segment (start 117.45 96.584321) (end 117.45 111) (width 0.25) (layer "F.Cu") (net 28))
 (segment (start 116.359449 95.49377) (end 117.45 96.584321) (width 0.25) (layer "F.Cu") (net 28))
 (segment (start 118 96.427215) (end 118 110.913604) (width 0.25) (layer "F.Cu") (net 29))
 (segment (start 118 110.913604) (end 118.846396 111.76) (width 0.25) (layer "F.Cu") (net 29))
 (segment (start 116.713002 95.140217) (end 118 96.427215) (width 0.25) (layer "F.Cu") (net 29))
 (segment (start 118.846396 111.76) (end 124.46 111.76) (width 0.25) (layer "F.Cu") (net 29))
 (segment (start 118.45 107.45) (end 120.22 109.22) (width 0.25) (layer "F.Cu") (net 30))
 (segment (start 120.22 109.22) (end 124.46 109.22) (width 0.25) (layer "F.Cu") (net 30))
 (segment (start 118.45 96.170109) (end 118.45 107.45) (width 0.25) (layer "F.Cu") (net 30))
 (segment (start 117.066555 94.786664) (end 118.45 96.170109) (width 0.25) (layer "F.Cu") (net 30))
 (segment (start 119 96.013001) (end 119 105) (width 0.25) (layer "F.Cu") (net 31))
 (segment (start 119 105) (end 120.68 106.68) (width 0.25) (layer "F.Cu") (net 31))
 (segment (start 120.68 106.68) (end 124.46 106.68) (width 0.25) (layer "F.Cu") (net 31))
 (segment (start 117.420109 94.43311) (end 119 96.013001) (width 0.25) (layer "F.Cu") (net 31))
 (segment (start 117.773662 94.079557) (end 119.311698 95.617593) (width 0.25) (layer "F.Cu") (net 32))
 (segment (start 123.32 103) (end 124.46 104.14) (width 0.25) (layer "F.Cu") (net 32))
 (segment (start 119.45 103) (end 123.32 103) (width 0.25) (layer "F.Cu") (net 32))
 (segment (start 119.311698 95.617593) (end 119.311698 95.688303) (width 0.25) (layer "F.Cu") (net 32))
 (segment (start 119.311698 95.688303) (end 119.45 95.826605) (width 0.25) (layer "F.Cu") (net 32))
 (segment (start 119.45 95.826605) (end 119.45 103) (width 0.25) (layer "F.Cu") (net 32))
 (segment (start 118.127215 93.726004) (end 120 95.598789) (width 0.25) (layer "F.Cu") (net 33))
 (segment (start 120 95.598789) (end 120 100) (width 0.25) (layer "F.Cu") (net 33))
 (segment (start 120 100) (end 121.6 101.6) (width 0.25) (layer "F.Cu") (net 33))
 (segment (start 121.6 101.6) (end 124.46 101.6) (width 0.25) (layer "F.Cu") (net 33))
 (segment (start 120.45 95.341681) (end 120.45 98) (width 0.25) (layer "F.Cu") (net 34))
 (segment (start 123.4 98) (end 124.46 99.06) (width 0.25) (layer "F.Cu") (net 34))
 (segment (start 120.45 98) (end 123.4 98) (width 0.25) (layer "F.Cu") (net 34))
 (segment (start 118.480769 93.37245) (end 120.45 95.341681) (width 0.25) (layer "F.Cu") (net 34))
 (segment (start 121 95.184575) (end 121 96) (width 0.25) (layer "F.Cu") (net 35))
 (segment (start 121 96) (end 121.52 96.52) (width 0.25) (layer "F.Cu") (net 35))
 (segment (start 121.52 96.52) (end 124.46 96.52) (width 0.25) (layer "F.Cu") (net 35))
 (segment (start 118.834322 93.018897) (end 121 95.184575) (width 0.25) (layer "F.Cu") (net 35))
 (segment (start 119.187876 92.665343) (end 119.665343 92.665343) (width 0.25) (layer "F.Cu") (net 36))
 (segment (start 119.665343 92.665343) (end 121 94) (width 0.25) (layer "F.Cu") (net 36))
 (segment (start 121.02 93.98) (end 124.46 93.98) (width 0.25) (layer "F.Cu") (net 36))
 (segment (start 121 94) (end 121.02 93.98) (width 0.25) (layer "F.Cu") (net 36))
 (segment (start 119.187876 90.667767) (end 123.687767 90.667767) (width 0.25) (layer "F.Cu") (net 37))
 (segment (start 123.687767 90.667767) (end 124.46 91.44) (width 0.25) (layer "F.Cu") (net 37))
 (segment (start 118.834322 90.314213) (end 120.248535 88.9) (width 0.25) (layer "F.Cu") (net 38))
 (segment (start 120.248535 88.9) (end 124.46 88.9) (width 0.25) (layer "F.Cu") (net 38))
 (segment (start 122.081429 86.36) (end 124.46 86.36) (width 0.25) (layer "F.Cu") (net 39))
 (segment (start 118.480769 89.96066) (end 122.081429 86.36) (width 0.25) (layer "F.Cu") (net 39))
 (segment (start 118.127215 89.607106) (end 123.914321 83.82) (width 0.25) (layer "F.Cu") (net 40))
 (segment (start 123.914321 83.82) (end 124.46 83.82) (width 0.25) (layer "F.Cu") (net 40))
 (segment (start 123.285 83.742215) (end 123.285 82.455) (width 0.25) (layer "F.Cu") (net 41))
 (segment (start 117.773662 89.253553) (end 123.285 83.742215) (width 0.25) (layer "F.Cu") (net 41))
 (segment (start 123.285 82.455) (end 124.46 81.28) (width 0.25) (layer "F.Cu") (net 41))
 (segment (start 117.420109 88.9) (end 122.835 83.485109) (width 0.25) (layer "F.Cu") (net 42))
 (segment (start 122.835 83.485109) (end 122.835 80.365) (width 0.25) (layer "F.Cu") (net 42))
 (segment (start 122.835 80.365) (end 124.46 78.74) (width 0.25) (layer "F.Cu") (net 42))
 (segment (start 122 78.66) (end 124.46 76.2) (width 0.25) (layer "F.Cu") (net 43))
 (segment (start 122 83.613001) (end 122 78.66) (width 0.25) (layer "F.Cu") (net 43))
 (segment (start 117.066555 88.546446) (end 122 83.613001) (width 0.25) (layer "F.Cu") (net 43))
 (segment (start 116.713002 88.192893) (end 116.748356 88.192893) (width 0.25) (layer "F.Cu") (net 44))
 (segment (start 121.55 76.57) (end 124.46 73.66) (width 0.25) (layer "F.Cu") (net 44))
 (segment (start 116.748356 88.192893) (end 121.55 83.391249) (width 0.25) (layer "F.Cu") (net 44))
 (segment (start 121.55 83.391249) (end 121.55 76.57) (width 0.25) (layer "F.Cu") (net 44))
 (segment (start 116.359449 87.83934) (end 121 83.198789) (width 0.25) (layer "F.Cu") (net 45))
 (segment (start 121 83.198789) (end 121 74.58) (width 0.25) (layer "F.Cu") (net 45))
 (segment (start 121 74.58) (end 124.46 71.12) (width 0.25) (layer "F.Cu") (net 45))
 (segment (start 120.971802 72.068198) (end 124.46 68.58) (width 0.25) (layer "F.Cu") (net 46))
 (segment (start 116.005895 87.485786) (end 120.55 82.941681) (width 0.25) (layer "F.Cu") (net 46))
 (segment (start 120.971802 73.971802) (end 120.971802 72.068198) (width 0.25) (layer "F.Cu") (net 46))
 (segment (start 120.55 82.941681) (end 120.55 74.393604) (width 0.25) (layer "F.Cu") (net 46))
 (segment (start 120.55 74.393604) (end 120.971802 73.971802) (width 0.25) (layer "F.Cu") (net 46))
 (segment (start 122 69) (end 122 68.5) (width 0.25) (layer "F.Cu") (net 47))
 (segment (start 116.221749 86.562826) (end 116.292459 86.562826) (width 0.25) (layer "F.Cu") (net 47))
 (segment (start 115.652342 87.132233) (end 116.221749 86.562826) (width 0.25) (layer "F.Cu") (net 47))
 (segment (start 119.927643 71.072357) (end 122 69) (width 0.25) (layer "F.Cu") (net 47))
 (segment (start 119.927643 82.927642) (end 119.927643 71.072357) (width 0.25) (layer "F.Cu") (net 47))
 (segment (start 122 68.5) (end 124.46 66.04) (width 0.25) (layer "F.Cu") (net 47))
 (segment (start 116.292459 86.562826) (end 119.927643 82.927642) (width 0.25) (layer "F.Cu") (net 47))
 (segment (start 120 69) (end 120 67.96) (width 0.25) (layer "F.Cu") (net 48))
 (segment (start 115.298788 86.778679) (end 119 83.077467) (width 0.25) (layer "F.Cu") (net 48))
 (segment (start 120 67.96) (end 124.46 63.5) (width 0.25) (layer "F.Cu") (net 48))
 (segment (start 119 83.077467) (end 119 83) (width 0.25) (layer "F.Cu") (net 48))
 (segment (start 119.477643 82.599824) (end 119.477643 69.522357) (width 0.25) (layer "F.Cu") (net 48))
 (segment (start 119.477643 69.522357) (end 120 69) (width 0.25) (layer "F.Cu") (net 48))
 (segment (start 119 83.077467) (end 119.477643 82.599824) (width 0.25) (layer "F.Cu") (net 48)))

